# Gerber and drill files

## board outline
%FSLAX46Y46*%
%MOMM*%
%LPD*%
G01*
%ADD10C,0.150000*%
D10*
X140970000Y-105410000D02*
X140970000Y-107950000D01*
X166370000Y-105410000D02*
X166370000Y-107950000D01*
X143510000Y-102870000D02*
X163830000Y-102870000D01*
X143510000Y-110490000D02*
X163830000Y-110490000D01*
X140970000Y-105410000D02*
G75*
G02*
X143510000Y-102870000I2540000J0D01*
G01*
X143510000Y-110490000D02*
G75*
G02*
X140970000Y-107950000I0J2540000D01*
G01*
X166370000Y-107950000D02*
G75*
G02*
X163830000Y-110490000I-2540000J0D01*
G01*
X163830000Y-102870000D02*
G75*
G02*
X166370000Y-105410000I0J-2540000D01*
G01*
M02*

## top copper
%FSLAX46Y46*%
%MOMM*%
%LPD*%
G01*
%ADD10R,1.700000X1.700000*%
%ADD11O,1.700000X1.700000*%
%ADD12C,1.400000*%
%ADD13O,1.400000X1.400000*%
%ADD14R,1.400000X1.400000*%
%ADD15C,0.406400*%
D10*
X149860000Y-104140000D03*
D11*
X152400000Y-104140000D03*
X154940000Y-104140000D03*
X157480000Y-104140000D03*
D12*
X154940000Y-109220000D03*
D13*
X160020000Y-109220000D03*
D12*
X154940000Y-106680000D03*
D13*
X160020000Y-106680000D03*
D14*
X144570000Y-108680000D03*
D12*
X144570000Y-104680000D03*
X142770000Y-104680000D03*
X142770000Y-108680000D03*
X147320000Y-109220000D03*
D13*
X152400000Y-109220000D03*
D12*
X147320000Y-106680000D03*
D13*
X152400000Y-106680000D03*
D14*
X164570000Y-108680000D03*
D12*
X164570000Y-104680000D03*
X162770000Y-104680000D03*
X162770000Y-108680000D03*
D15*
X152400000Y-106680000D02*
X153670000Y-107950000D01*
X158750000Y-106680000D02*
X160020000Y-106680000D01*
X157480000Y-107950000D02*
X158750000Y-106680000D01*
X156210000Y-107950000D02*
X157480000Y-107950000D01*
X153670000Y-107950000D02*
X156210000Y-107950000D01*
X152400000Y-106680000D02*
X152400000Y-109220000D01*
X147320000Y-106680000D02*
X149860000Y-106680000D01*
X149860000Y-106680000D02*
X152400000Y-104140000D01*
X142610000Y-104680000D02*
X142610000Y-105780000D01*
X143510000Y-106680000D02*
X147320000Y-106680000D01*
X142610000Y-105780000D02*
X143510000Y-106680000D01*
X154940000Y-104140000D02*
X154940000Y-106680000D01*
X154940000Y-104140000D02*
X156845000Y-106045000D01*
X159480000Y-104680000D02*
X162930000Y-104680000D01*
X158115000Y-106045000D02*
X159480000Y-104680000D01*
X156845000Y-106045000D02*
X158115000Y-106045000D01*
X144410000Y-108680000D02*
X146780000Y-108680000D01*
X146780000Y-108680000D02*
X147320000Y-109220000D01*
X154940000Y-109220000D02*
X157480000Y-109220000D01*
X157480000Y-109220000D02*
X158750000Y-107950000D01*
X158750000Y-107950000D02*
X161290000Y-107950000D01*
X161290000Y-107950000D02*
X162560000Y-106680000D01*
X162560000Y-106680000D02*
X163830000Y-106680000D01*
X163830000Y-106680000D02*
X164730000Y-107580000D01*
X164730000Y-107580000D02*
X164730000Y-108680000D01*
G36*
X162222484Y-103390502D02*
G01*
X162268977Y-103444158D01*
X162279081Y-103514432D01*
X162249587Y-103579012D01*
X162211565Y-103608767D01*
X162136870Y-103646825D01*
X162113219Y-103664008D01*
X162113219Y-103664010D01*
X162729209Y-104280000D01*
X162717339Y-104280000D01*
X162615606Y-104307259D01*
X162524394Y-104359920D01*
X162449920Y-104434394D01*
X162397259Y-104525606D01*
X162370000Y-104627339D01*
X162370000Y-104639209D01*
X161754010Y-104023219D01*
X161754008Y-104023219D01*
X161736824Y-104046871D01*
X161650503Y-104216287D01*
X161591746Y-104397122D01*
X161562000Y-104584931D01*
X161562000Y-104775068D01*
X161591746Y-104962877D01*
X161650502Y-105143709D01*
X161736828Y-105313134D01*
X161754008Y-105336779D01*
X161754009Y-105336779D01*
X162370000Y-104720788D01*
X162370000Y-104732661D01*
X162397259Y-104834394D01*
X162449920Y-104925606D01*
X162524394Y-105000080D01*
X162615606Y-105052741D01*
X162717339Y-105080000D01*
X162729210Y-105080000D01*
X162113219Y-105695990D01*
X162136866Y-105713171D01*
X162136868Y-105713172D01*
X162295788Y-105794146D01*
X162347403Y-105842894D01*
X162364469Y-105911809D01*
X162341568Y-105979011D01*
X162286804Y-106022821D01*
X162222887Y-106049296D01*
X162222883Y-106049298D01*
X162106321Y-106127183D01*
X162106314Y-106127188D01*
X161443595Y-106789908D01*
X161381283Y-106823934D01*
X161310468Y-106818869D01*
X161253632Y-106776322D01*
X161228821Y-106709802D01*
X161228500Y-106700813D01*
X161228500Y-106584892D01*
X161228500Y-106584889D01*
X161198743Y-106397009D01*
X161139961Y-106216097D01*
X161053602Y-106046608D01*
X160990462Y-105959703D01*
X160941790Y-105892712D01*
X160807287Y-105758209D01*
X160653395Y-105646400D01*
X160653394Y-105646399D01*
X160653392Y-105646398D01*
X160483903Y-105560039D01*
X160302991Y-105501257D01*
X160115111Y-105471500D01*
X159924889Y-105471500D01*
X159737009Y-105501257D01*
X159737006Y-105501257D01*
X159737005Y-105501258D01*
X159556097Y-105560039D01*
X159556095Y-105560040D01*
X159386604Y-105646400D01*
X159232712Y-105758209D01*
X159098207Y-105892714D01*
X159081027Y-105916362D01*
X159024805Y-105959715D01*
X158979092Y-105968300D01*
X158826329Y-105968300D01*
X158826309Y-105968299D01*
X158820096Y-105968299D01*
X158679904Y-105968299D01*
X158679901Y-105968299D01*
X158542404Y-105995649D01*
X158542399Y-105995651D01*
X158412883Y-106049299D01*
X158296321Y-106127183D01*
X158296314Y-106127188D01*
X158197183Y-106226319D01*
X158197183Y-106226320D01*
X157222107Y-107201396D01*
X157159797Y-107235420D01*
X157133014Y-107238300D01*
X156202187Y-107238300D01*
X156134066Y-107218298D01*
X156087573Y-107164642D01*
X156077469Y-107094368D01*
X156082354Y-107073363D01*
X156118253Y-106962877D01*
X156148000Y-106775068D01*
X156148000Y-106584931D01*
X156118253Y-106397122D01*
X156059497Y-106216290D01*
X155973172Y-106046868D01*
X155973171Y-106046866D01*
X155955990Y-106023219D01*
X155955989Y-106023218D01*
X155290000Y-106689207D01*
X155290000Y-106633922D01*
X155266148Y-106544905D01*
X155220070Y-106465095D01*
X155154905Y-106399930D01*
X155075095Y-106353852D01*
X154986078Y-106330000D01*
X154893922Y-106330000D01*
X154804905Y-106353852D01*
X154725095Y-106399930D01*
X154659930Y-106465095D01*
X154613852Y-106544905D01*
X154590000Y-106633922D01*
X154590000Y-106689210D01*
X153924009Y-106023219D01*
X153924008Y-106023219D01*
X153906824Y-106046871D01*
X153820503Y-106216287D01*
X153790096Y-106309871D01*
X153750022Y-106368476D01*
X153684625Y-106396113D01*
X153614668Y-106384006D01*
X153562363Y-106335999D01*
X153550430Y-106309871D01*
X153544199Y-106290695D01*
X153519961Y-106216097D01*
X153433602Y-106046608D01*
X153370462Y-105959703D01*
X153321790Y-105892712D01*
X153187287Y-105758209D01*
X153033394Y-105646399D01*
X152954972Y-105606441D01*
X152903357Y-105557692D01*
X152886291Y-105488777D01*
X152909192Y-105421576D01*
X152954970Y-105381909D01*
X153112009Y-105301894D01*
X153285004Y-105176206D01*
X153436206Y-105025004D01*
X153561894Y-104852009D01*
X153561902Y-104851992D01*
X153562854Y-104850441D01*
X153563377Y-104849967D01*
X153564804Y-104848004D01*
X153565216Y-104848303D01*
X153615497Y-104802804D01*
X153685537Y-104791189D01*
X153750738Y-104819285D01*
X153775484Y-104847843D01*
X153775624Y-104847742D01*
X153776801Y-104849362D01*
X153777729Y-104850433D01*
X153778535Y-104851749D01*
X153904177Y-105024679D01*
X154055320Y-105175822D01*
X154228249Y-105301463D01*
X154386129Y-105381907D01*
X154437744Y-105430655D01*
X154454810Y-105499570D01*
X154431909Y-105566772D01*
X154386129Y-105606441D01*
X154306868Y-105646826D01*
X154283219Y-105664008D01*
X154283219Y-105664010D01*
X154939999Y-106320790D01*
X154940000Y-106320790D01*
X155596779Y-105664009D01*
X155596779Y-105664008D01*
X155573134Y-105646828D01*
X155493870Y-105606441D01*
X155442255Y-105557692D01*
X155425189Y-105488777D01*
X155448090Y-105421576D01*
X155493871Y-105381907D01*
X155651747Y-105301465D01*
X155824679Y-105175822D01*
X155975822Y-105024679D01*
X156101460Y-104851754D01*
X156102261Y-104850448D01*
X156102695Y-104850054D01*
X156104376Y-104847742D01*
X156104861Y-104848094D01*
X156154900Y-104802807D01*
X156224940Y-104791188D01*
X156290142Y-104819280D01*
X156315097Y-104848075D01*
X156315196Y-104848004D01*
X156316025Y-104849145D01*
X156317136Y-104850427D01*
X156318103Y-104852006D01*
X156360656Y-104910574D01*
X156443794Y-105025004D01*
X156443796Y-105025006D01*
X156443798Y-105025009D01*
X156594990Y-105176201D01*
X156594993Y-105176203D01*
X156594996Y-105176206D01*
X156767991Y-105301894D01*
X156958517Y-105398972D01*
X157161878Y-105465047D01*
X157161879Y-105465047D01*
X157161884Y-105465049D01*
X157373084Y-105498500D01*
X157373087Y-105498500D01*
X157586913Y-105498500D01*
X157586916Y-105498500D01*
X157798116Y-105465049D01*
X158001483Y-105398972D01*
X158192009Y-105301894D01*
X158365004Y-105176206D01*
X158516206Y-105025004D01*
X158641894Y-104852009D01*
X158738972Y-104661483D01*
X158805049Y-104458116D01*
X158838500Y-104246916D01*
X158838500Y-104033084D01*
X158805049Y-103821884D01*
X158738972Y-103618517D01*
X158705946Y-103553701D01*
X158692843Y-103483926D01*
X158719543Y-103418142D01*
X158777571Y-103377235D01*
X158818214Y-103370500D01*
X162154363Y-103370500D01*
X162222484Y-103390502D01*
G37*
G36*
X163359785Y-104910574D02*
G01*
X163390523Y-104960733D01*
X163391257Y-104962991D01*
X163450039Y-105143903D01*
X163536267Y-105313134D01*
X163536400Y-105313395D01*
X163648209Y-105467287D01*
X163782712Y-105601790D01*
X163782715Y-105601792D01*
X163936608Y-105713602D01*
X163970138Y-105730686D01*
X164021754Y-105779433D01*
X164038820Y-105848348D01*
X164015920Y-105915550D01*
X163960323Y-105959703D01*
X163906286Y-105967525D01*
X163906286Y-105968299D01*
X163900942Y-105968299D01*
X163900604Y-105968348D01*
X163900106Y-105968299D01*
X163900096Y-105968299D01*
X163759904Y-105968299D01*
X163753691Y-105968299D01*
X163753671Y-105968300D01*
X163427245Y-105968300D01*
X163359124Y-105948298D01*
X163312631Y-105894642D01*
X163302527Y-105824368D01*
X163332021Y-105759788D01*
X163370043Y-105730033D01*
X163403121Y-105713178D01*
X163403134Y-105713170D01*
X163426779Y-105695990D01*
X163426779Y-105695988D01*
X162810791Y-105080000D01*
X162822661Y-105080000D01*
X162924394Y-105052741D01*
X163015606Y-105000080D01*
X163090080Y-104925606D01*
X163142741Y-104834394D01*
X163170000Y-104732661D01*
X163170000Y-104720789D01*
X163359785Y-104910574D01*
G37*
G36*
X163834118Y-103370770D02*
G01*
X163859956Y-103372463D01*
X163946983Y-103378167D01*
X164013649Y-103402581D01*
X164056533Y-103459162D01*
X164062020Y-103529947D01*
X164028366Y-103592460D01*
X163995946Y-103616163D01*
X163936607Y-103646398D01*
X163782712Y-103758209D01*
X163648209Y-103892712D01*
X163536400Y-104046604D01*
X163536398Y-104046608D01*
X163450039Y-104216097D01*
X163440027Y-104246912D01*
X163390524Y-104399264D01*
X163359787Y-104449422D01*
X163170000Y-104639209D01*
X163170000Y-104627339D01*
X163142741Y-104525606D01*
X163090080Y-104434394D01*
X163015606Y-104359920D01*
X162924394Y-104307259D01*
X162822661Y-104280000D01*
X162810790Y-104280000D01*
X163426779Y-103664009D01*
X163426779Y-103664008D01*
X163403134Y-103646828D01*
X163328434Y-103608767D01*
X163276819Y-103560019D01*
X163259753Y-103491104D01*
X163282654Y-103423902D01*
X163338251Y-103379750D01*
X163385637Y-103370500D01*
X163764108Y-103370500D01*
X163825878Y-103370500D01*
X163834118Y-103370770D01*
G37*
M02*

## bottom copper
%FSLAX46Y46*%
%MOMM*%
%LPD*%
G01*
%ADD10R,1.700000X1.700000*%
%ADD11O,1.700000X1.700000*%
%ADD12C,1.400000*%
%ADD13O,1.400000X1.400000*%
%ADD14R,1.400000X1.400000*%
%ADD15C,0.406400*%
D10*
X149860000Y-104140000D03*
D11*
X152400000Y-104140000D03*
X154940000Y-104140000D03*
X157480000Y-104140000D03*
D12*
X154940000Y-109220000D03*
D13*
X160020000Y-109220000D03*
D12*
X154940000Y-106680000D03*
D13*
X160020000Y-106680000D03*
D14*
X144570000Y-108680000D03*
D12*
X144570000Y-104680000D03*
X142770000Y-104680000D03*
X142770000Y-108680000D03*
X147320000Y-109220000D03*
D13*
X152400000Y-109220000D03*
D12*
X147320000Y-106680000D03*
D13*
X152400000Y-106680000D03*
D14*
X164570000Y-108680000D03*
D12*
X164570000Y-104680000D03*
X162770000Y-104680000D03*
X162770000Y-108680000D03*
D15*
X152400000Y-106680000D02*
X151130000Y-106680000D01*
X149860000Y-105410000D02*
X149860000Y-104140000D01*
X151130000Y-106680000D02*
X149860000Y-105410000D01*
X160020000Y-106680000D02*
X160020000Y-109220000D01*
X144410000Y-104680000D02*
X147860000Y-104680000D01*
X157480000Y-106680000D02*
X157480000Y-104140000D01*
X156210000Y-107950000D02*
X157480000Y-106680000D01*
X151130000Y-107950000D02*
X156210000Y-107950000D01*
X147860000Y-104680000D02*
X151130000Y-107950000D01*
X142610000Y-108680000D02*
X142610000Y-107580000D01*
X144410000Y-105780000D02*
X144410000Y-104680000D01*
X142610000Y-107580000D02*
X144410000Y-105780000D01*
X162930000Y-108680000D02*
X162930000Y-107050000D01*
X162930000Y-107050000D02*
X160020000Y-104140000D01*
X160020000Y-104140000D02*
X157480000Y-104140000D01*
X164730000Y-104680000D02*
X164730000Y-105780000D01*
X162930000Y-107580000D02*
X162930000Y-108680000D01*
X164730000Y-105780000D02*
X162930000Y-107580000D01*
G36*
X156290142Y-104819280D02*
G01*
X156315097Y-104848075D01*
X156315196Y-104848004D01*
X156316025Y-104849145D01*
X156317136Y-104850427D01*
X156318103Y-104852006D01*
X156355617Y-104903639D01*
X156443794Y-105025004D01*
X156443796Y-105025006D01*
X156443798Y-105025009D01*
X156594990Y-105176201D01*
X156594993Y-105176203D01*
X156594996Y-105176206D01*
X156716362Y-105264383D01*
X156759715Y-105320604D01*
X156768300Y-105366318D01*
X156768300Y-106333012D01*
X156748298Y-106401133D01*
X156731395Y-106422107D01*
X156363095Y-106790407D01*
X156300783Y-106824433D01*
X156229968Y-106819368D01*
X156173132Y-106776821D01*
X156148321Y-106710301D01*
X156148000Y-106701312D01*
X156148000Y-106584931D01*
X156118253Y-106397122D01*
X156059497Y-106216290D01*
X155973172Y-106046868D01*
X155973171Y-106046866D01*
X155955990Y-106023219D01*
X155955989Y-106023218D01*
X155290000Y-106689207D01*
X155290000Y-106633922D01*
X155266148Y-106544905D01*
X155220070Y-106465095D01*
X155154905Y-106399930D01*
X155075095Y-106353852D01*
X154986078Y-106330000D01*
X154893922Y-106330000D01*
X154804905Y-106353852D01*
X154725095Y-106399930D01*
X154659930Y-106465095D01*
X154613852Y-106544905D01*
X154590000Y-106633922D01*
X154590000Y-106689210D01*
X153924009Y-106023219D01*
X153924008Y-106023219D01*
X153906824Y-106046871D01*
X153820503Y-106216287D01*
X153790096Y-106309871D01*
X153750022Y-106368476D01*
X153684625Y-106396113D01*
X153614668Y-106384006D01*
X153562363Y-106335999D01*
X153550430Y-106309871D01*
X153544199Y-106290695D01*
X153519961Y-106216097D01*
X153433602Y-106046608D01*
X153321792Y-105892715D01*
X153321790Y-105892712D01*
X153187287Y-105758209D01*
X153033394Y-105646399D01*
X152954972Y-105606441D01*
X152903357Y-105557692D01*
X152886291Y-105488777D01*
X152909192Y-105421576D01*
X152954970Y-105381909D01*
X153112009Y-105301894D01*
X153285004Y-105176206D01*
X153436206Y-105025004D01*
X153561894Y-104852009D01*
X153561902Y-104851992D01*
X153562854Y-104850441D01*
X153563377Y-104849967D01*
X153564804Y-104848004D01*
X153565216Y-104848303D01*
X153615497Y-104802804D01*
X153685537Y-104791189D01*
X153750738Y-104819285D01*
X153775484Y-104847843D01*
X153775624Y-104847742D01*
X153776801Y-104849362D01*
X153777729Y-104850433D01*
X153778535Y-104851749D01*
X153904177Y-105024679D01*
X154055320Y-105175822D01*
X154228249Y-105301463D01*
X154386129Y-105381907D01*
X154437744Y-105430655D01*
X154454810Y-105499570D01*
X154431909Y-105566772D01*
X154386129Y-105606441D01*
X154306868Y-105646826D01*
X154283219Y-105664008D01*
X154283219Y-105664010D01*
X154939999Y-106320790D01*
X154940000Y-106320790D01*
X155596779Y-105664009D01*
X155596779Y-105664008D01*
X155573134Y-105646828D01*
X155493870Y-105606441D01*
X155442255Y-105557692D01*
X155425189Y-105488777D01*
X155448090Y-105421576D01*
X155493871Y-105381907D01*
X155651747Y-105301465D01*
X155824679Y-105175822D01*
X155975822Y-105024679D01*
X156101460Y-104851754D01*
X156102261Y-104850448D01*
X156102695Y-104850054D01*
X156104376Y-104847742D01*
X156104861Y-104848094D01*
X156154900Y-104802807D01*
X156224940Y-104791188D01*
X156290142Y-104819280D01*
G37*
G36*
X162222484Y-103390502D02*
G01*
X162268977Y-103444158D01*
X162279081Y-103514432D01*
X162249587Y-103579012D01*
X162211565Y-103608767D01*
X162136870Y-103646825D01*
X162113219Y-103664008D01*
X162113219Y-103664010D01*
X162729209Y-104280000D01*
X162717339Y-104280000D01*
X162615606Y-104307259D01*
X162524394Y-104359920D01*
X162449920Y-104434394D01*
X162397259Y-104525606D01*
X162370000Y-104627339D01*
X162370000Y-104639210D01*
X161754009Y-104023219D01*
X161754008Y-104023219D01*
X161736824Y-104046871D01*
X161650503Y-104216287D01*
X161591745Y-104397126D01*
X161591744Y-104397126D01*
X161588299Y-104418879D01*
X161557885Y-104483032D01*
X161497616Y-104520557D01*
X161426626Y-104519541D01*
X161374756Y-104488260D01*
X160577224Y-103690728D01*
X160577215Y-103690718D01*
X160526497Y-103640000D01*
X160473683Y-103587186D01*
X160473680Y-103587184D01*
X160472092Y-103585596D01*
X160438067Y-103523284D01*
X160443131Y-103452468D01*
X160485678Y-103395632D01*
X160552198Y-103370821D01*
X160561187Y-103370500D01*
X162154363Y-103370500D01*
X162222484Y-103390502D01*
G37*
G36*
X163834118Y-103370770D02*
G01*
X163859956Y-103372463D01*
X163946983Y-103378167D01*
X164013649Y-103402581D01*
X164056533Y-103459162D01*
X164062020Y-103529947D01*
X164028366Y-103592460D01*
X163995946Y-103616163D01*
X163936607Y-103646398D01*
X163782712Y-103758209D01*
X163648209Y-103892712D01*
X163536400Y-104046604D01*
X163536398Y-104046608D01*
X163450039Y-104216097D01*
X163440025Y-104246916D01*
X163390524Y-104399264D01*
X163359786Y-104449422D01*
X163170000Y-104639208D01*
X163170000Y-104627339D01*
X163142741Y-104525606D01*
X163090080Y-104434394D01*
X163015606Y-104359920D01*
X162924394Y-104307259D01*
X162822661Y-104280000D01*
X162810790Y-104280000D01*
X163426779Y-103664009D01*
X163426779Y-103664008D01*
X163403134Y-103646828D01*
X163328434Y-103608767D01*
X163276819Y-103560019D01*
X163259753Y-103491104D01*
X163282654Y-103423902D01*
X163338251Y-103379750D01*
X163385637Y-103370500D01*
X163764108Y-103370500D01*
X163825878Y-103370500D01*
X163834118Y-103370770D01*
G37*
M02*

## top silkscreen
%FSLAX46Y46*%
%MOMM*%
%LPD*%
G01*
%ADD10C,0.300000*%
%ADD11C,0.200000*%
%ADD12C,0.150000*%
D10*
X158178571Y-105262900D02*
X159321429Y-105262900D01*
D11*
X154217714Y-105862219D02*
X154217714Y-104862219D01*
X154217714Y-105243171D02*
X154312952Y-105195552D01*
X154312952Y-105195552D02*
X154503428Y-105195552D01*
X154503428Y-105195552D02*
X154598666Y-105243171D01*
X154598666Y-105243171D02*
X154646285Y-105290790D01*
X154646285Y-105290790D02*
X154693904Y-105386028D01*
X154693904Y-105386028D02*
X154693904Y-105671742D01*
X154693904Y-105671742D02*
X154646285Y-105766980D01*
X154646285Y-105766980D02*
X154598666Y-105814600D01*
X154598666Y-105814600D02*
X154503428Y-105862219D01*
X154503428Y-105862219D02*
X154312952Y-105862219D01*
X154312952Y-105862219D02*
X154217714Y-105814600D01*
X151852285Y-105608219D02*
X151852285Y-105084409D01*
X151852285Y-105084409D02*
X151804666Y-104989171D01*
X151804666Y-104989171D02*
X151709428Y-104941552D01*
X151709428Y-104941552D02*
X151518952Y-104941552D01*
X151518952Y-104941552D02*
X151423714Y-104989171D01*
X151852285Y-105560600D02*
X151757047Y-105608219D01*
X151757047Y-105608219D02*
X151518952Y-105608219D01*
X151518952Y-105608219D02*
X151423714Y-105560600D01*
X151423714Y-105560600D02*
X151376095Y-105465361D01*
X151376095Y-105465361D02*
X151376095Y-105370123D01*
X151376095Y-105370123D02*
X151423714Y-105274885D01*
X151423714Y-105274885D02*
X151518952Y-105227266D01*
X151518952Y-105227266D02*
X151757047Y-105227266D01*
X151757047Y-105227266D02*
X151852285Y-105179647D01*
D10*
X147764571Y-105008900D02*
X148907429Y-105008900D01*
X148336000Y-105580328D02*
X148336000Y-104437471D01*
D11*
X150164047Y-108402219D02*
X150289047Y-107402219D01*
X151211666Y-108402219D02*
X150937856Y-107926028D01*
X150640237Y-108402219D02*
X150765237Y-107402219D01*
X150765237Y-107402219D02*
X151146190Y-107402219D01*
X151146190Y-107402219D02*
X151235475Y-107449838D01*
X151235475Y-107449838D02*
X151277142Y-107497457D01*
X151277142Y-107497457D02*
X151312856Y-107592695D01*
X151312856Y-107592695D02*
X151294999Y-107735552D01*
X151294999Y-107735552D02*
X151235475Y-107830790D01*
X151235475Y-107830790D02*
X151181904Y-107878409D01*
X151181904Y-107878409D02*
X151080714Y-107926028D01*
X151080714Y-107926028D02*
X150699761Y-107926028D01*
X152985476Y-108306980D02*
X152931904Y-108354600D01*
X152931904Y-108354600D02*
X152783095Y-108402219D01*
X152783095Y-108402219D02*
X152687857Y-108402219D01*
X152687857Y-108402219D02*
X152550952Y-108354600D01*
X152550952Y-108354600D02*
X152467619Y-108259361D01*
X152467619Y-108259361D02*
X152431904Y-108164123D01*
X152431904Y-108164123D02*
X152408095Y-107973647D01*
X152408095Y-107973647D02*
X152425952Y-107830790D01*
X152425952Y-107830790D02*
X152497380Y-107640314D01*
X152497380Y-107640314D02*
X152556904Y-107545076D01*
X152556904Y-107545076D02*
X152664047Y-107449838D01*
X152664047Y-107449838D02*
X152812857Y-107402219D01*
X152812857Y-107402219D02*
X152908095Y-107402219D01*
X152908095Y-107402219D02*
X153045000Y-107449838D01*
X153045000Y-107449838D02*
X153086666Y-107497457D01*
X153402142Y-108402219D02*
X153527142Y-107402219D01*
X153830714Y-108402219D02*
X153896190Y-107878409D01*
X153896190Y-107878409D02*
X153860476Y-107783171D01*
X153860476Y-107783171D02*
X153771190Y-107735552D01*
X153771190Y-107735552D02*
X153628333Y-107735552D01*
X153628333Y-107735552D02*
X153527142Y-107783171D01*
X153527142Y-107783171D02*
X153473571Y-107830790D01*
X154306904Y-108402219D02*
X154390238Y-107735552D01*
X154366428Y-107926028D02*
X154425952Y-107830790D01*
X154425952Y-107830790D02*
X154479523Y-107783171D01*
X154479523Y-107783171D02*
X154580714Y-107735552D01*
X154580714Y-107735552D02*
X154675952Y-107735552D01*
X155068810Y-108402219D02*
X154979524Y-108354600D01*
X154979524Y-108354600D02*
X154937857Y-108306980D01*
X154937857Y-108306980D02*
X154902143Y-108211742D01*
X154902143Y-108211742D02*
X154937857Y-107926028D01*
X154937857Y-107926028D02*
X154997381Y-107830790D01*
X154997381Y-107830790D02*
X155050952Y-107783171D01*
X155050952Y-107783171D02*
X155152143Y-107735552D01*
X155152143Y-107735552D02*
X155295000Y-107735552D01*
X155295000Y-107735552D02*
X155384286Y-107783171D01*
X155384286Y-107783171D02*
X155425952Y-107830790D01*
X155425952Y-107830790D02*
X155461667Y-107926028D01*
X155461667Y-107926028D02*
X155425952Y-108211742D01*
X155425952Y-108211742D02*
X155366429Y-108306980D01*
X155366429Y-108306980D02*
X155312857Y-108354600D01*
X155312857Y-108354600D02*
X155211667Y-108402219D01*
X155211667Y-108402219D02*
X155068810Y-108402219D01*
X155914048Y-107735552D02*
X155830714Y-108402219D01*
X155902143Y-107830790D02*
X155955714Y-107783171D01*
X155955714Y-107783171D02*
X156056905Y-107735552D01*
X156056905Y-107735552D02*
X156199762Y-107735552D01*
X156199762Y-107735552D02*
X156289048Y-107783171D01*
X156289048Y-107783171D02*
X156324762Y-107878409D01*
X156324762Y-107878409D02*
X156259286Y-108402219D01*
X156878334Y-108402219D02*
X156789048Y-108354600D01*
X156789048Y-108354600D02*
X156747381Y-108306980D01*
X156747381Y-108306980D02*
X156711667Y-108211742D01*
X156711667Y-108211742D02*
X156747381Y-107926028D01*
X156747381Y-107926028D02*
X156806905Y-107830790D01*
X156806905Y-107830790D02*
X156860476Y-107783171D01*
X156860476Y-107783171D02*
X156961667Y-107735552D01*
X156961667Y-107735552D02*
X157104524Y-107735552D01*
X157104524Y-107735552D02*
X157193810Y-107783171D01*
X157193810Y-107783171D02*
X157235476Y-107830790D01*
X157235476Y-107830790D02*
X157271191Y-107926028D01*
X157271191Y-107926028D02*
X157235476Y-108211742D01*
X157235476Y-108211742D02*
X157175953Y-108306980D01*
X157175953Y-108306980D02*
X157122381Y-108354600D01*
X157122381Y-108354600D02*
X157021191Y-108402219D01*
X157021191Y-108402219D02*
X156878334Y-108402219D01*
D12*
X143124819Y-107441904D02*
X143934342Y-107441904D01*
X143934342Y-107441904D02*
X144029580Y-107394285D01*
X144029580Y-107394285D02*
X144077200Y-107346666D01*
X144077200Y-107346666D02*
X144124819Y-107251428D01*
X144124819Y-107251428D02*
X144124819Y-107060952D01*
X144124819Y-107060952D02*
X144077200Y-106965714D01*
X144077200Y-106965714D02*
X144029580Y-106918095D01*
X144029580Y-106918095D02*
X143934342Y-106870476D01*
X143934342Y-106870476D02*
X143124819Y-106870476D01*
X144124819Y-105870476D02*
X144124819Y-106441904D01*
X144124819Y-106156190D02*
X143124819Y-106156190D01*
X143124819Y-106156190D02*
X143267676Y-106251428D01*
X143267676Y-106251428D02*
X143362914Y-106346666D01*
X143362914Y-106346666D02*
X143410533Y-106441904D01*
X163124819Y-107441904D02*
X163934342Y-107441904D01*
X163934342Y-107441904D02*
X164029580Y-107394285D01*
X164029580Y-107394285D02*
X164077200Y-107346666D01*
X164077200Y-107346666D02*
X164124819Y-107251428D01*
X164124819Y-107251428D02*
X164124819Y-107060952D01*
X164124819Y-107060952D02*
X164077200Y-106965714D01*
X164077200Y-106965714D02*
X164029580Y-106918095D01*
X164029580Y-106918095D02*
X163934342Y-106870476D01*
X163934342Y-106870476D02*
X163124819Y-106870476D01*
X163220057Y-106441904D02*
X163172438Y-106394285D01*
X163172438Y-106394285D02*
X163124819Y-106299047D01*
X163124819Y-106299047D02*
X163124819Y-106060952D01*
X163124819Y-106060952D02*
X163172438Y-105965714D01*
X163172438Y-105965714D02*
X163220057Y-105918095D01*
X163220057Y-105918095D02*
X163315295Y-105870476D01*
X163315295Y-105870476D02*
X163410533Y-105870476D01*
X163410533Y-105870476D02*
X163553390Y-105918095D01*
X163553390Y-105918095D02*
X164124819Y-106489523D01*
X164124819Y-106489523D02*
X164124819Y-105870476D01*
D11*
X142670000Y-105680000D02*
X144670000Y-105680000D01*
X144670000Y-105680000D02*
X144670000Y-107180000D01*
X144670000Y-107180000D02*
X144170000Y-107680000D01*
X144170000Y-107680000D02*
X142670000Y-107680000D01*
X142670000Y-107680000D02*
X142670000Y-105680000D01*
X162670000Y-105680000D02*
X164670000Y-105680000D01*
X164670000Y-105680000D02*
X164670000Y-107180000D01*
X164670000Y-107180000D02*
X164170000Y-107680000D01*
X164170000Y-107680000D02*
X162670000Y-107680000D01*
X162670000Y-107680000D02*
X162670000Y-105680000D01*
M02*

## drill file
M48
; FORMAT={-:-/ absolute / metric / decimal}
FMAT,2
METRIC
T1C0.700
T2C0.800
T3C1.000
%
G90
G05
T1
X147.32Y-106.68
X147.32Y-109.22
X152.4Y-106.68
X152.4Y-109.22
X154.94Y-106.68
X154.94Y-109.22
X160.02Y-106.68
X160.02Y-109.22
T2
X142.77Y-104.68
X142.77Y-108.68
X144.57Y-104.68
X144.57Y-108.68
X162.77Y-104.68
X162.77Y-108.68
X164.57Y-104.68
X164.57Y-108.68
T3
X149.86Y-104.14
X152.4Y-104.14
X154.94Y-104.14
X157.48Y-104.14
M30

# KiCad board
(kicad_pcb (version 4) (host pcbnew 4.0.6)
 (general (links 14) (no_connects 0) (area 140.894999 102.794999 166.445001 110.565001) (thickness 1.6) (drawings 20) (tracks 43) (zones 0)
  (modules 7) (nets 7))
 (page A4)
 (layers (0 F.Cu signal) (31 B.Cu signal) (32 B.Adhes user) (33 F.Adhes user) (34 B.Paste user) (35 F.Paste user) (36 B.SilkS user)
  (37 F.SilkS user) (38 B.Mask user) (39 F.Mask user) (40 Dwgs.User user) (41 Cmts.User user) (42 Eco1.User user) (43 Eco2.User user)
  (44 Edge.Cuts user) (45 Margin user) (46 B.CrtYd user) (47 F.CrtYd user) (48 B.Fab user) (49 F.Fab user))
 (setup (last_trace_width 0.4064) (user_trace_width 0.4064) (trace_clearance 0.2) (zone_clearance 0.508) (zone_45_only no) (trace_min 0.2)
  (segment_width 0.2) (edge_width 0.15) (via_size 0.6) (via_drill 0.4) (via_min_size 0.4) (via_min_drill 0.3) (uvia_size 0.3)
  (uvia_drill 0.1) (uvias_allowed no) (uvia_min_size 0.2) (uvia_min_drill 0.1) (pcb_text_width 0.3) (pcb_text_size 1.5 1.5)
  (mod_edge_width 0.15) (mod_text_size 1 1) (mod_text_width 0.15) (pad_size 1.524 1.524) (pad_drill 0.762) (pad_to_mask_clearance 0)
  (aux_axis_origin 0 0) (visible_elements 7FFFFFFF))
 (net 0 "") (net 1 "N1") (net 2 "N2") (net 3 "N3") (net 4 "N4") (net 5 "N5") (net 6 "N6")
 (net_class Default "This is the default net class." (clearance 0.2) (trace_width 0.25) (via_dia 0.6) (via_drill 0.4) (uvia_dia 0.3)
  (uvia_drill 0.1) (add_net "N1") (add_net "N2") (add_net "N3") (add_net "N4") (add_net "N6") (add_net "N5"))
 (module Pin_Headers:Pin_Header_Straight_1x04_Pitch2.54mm (layer F.Cu) (at 149.86 104.14 90)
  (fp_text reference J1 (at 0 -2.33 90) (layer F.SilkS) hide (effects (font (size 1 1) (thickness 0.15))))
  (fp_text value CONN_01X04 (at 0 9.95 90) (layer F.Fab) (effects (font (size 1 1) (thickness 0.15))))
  (pad 1 thru_hole rect (at 0 0 90) (size 1.7 1.7) (drill 1) (layers *.Cu *.Mask) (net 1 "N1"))
  (pad 2 thru_hole oval (at 0 2.54 90) (size 1.7 1.7) (drill 1) (layers *.Cu *.Mask) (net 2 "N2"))
  (pad 3 thru_hole oval (at 0 5.08 90) (size 1.7 1.7) (drill 1) (layers *.Cu *.Mask) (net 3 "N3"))
  (pad 4 thru_hole oval (at 0 7.62 90) (size 1.7 1.7) (drill 1) (layers *.Cu *.Mask) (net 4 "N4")))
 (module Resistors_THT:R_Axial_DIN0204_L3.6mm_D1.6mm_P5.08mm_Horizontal (layer B.Cu) (at 154.94 109.22)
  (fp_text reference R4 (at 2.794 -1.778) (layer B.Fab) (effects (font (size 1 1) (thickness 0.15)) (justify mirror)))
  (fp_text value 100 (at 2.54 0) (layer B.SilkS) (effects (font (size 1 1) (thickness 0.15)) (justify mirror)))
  (pad 1 thru_hole circle (at 0 0) (size 1.4 1.4) (drill 0.7) (layers *.Cu *.Mask) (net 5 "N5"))
  (pad 2 thru_hole oval (at 5.08 0) (size 1.4 1.4) (drill 0.7) (layers *.Cu *.Mask) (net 1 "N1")))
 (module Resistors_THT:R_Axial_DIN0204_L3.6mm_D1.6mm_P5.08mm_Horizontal (layer B.Cu) (at 154.94 106.68)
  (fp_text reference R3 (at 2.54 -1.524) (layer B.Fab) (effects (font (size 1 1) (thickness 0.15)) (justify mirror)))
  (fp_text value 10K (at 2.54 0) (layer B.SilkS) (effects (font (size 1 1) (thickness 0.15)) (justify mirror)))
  (pad 1 thru_hole circle (at 0 0) (size 1.4 1.4) (drill 0.7) (layers *.Cu *.Mask) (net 3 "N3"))
  (pad 2 thru_hole oval (at 5.08 0) (size 1.4 1.4) (drill 0.7) (layers *.Cu *.Mask) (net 1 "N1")))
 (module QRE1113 (layer F.Cu) (at 143.67 106.68 90)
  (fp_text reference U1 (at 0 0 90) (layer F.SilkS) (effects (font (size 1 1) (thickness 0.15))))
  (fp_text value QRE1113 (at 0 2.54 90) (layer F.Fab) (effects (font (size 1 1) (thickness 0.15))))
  (fp_line (start 1 -1) (end 1 1) (layer F.SilkS) (width 0.2))
  (fp_line (start 1 1) (end -0.5 1) (layer F.SilkS) (width 0.2))
  (fp_line (start -0.5 1) (end -1 0.5) (layer F.SilkS) (width 0.2))
  (fp_line (start -1 0.5) (end -1 -1) (layer F.SilkS) (width 0.2))
  (fp_line (start -1 -1) (end 1 -1) (layer F.SilkS) (width 0.2))
  (pad 1 thru_hole rect (at -2 0.9 90) (size 1.4 1.4) (drill 0.8) (layers *.Cu *.Mask) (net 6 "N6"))
  (pad 2 thru_hole circle (at 2 0.9 90) (size 1.4 1.4) (drill 0.8) (layers *.Cu *.Mask) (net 4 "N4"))
  (pad 3 thru_hole circle (at 2 -0.9 90) (size 1.4 1.4) (drill 0.8) (layers *.Cu *.Mask) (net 2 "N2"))
  (pad 4 thru_hole circle (at -2 -0.9 90) (size 1.4 1.4) (drill 0.8) (layers *.Cu *.Mask) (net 4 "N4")))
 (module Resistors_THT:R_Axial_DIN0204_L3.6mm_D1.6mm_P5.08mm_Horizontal (layer B.Cu) (at 147.32 109.22)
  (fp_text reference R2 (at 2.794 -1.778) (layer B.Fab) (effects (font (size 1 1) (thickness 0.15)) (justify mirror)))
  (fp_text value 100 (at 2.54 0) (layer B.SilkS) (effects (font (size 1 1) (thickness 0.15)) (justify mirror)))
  (pad 1 thru_hole circle (at 0 0) (size 1.4 1.4) (drill 0.7) (layers *.Cu *.Mask) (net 6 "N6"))
  (pad 2 thru_hole oval (at 5.08 0) (size 1.4 1.4) (drill 0.7) (layers *.Cu *.Mask) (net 1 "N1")))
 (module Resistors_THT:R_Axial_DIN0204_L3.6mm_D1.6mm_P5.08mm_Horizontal (layer B.Cu) (at 147.32 106.68)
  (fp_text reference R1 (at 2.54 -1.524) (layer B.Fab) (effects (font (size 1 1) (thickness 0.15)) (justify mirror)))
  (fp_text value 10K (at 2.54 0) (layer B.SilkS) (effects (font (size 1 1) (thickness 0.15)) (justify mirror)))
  (pad 1 thru_hole circle (at 0 0) (size 1.4 1.4) (drill 0.7) (layers *.Cu *.Mask) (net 2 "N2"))
  (pad 2 thru_hole oval (at 5.08 0) (size 1.4 1.4) (drill 0.7) (layers *.Cu *.Mask) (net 1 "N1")))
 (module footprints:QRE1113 (layer F.Cu) (at 163.67 106.68 90)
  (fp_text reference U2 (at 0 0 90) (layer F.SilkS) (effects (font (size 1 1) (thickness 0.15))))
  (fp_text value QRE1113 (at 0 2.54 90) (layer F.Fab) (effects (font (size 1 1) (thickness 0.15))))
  (fp_line (start 1 -1) (end 1 1) (layer F.SilkS) (width 0.2))
  (fp_line (start 1 1) (end -0.5 1) (layer F.SilkS) (width 0.2))
  (fp_line (start -0.5 1) (end -1 0.5) (layer F.SilkS) (width 0.2))
  (fp_line (start -1 0.5) (end -1 -1) (layer F.SilkS) (width 0.2))
  (fp_line (start -1 -1) (end 1 -1) (layer F.SilkS) (width 0.2))
  (pad 1 thru_hole rect (at -2 0.9 90) (size 1.4 1.4) (drill 0.8) (layers *.Cu *.Mask) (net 5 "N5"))
  (pad 2 thru_hole circle (at 2 0.9 90) (size 1.4 1.4) (drill 0.8) (layers *.Cu *.Mask) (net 4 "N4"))
  (pad 3 thru_hole circle (at 2 -0.9 90) (size 1.4 1.4) (drill 0.8) (layers *.Cu *.Mask) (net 3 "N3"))
  (pad 4 thru_hole circle (at -2 -0.9 90) (size 1.4 1.4) (drill 0.8) (layers *.Cu *.Mask) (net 4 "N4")))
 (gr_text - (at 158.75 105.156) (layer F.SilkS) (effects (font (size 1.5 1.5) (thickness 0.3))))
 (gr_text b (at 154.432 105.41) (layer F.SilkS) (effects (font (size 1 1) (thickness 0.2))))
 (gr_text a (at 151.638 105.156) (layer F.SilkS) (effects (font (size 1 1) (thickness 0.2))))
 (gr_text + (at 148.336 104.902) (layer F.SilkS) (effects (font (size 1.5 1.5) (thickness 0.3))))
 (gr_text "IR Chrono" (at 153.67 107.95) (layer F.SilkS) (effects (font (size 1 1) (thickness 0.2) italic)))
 (gr_line (start 140.97 105.41) (end 140.97 107.95) (angle 90) (layer Edge.Cuts) (width 0.15))
 (gr_line (start 166.37 105.41) (end 166.37 107.95) (angle 90) (layer Edge.Cuts) (width 0.15))
 (gr_line (start 143.51 102.87) (end 163.83 102.87) (angle 90) (layer Edge.Cuts) (width 0.15))
 (gr_line (start 143.51 110.49) (end 163.83 110.49) (angle 90) (layer Edge.Cuts) (width 0.15))
 (gr_arc (start 143.51 105.41) (end 140.97 105.41) (angle 90) (layer Edge.Cuts) (width 0.15))
 (gr_arc (start 143.51 107.95) (end 143.51 110.49) (angle 90) (layer Edge.Cuts) (width 0.15))
 (gr_arc (start 163.83 107.95) (end 166.37 107.95) (angle 90) (layer Edge.Cuts) (width 0.15))
 (gr_arc (start 163.83 105.41) (end 163.83 102.87) (angle 90) (layer Edge.Cuts) (width 0.15))
 (segment (start 152.4 106.68) (end 153.67 107.95) (width 0.4064) (layer F.Cu) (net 1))
 (segment (start 158.75 106.68) (end 160.02 106.68) (width 0.4064) (layer F.Cu) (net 1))
 (segment (start 157.48 107.95) (end 158.75 106.68) (width 0.4064) (layer F.Cu) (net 1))
 (segment (start 156.21 107.95) (end 157.48 107.95) (width 0.4064) (layer F.Cu) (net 1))
 (segment (start 153.67 107.95) (end 156.21 107.95) (width 0.4064) (layer F.Cu) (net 1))
 (segment (start 152.4 106.68) (end 152.4 109.22) (width 0.4064) (layer F.Cu) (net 1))
 (segment (start 152.4 106.68) (end 151.13 106.68) (width 0.4064) (layer B.Cu) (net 1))
 (segment (start 149.86 105.41) (end 149.86 104.14) (width 0.4064) (layer B.Cu) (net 1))
 (segment (start 151.13 106.68) (end 149.86 105.41) (width 0.4064) (layer B.Cu) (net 1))
 (segment (start 160.02 106.68) (end 160.02 109.22) (width 0.4064) (layer B.Cu) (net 1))
 (segment (start 147.32 106.68) (end 149.86 106.68) (width 0.4064) (layer F.Cu) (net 2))
 (segment (start 149.86 106.68) (end 152.4 104.14) (width 0.4064) (layer F.Cu) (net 2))
 (segment (start 142.61 104.68) (end 142.61 105.78) (width 0.4064) (layer F.Cu) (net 2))
 (segment (start 143.51 106.68) (end 147.32 106.68) (width 0.4064) (layer F.Cu) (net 2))
 (segment (start 142.61 105.78) (end 143.51 106.68) (width 0.4064) (layer F.Cu) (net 2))
 (segment (start 154.94 104.14) (end 154.94 106.68) (width 0.4064) (layer F.Cu) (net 3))
 (segment (start 154.94 104.14) (end 156.845 106.045) (width 0.4064) (layer F.Cu) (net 3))
 (segment (start 159.48 104.68) (end 162.93 104.68) (width 0.4064) (layer F.Cu) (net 3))
 (segment (start 158.115 106.045) (end 159.48 104.68) (width 0.4064) (layer F.Cu) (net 3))
 (segment (start 156.845 106.045) (end 158.115 106.045) (width 0.4064) (layer F.Cu) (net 3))
 (segment (start 144.41 108.68) (end 146.78 108.68) (width 0.4064) (layer F.Cu) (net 6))
 (segment (start 146.78 108.68) (end 147.32 109.22) (width 0.4064) (layer F.Cu) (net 6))
 (segment (start 154.94 109.22) (end 157.48 109.22) (width 0.4064) (layer F.Cu) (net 5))
 (segment (start 157.48 109.22) (end 158.75 107.95) (width 0.4064) (layer F.Cu) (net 5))
 (segment (start 158.75 107.95) (end 161.29 107.95) (width 0.4064) (layer F.Cu) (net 5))
 (segment (start 161.29 107.95) (end 162.56 106.68) (width 0.4064) (layer F.Cu) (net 5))
 (segment (start 162.56 106.68) (end 163.83 106.68) (width 0.4064) (layer F.Cu) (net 5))
 (segment (start 163.83 106.68) (end 164.73 107.58) (width 0.4064) (layer F.Cu) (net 5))
 (segment (start 164.73 107.58) (end 164.73 108.68) (width 0.4064) (layer F.Cu) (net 5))
 (segment (start 144.41 104.68) (end 147.86 104.68) (width 0.4064) (layer B.Cu) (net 4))
 (segment (start 157.48 106.68) (end 157.48 104.14) (width 0.4064) (layer B.Cu) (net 4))
 (segment (start 156.21 107.95) (end 157.48 106.68) (width 0.4064) (layer B.Cu) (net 4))
 (segment (start 151.13 107.95) (end 156.21 107.95) (width 0.4064) (layer B.Cu) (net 4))
 (segment (start 147.86 104.68) (end 151.13 107.95) (width 0.4064) (layer B.Cu) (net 4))
 (segment (start 142.61 108.68) (end 142.61 107.58) (width 0.4064) (layer B.Cu) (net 4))
 (segment (start 144.41 105.78) (end 144.41 104.68) (width 0.4064) (layer B.Cu) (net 4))
 (segment (start 142.61 107.58) (end 144.41 105.78) (width 0.4064) (layer B.Cu) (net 4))
 (segment (start 162.93 108.68) (end 162.93 107.05) (width 0.4064) (layer B.Cu) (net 4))
 (segment (start 162.93 107.05) (end 160.02 104.14) (width 0.4064) (layer B.Cu) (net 4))
 (segment (start 160.02 104.14) (end 157.48 104.14) (width 0.4064) (layer B.Cu) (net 4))
 (segment (start 164.73 104.68) (end 164.73 105.78) (width 0.4064) (layer B.Cu) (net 4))
 (segment (start 162.93 107.58) (end 162.93 108.68) (width 0.4064) (layer B.Cu) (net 4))
 (segment (start 164.73 105.78) (end 162.93 107.58) (width 0.4064) (layer B.Cu) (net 4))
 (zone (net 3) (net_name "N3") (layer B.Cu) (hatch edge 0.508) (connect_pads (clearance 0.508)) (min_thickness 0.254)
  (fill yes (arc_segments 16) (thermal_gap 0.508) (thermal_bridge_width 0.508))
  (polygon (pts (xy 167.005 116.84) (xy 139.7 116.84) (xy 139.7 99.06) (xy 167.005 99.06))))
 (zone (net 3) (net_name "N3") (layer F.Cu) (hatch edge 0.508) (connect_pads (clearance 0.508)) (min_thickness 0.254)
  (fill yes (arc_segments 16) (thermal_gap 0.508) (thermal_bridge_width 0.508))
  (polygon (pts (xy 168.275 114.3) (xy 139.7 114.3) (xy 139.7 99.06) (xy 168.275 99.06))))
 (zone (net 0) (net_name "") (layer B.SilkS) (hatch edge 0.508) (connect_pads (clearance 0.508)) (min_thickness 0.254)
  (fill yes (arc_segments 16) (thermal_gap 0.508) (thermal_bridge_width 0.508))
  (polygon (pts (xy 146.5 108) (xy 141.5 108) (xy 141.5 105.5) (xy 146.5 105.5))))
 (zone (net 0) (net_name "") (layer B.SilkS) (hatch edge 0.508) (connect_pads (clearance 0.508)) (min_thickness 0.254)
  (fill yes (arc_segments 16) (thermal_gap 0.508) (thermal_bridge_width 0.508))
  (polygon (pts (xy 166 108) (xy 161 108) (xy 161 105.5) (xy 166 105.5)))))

